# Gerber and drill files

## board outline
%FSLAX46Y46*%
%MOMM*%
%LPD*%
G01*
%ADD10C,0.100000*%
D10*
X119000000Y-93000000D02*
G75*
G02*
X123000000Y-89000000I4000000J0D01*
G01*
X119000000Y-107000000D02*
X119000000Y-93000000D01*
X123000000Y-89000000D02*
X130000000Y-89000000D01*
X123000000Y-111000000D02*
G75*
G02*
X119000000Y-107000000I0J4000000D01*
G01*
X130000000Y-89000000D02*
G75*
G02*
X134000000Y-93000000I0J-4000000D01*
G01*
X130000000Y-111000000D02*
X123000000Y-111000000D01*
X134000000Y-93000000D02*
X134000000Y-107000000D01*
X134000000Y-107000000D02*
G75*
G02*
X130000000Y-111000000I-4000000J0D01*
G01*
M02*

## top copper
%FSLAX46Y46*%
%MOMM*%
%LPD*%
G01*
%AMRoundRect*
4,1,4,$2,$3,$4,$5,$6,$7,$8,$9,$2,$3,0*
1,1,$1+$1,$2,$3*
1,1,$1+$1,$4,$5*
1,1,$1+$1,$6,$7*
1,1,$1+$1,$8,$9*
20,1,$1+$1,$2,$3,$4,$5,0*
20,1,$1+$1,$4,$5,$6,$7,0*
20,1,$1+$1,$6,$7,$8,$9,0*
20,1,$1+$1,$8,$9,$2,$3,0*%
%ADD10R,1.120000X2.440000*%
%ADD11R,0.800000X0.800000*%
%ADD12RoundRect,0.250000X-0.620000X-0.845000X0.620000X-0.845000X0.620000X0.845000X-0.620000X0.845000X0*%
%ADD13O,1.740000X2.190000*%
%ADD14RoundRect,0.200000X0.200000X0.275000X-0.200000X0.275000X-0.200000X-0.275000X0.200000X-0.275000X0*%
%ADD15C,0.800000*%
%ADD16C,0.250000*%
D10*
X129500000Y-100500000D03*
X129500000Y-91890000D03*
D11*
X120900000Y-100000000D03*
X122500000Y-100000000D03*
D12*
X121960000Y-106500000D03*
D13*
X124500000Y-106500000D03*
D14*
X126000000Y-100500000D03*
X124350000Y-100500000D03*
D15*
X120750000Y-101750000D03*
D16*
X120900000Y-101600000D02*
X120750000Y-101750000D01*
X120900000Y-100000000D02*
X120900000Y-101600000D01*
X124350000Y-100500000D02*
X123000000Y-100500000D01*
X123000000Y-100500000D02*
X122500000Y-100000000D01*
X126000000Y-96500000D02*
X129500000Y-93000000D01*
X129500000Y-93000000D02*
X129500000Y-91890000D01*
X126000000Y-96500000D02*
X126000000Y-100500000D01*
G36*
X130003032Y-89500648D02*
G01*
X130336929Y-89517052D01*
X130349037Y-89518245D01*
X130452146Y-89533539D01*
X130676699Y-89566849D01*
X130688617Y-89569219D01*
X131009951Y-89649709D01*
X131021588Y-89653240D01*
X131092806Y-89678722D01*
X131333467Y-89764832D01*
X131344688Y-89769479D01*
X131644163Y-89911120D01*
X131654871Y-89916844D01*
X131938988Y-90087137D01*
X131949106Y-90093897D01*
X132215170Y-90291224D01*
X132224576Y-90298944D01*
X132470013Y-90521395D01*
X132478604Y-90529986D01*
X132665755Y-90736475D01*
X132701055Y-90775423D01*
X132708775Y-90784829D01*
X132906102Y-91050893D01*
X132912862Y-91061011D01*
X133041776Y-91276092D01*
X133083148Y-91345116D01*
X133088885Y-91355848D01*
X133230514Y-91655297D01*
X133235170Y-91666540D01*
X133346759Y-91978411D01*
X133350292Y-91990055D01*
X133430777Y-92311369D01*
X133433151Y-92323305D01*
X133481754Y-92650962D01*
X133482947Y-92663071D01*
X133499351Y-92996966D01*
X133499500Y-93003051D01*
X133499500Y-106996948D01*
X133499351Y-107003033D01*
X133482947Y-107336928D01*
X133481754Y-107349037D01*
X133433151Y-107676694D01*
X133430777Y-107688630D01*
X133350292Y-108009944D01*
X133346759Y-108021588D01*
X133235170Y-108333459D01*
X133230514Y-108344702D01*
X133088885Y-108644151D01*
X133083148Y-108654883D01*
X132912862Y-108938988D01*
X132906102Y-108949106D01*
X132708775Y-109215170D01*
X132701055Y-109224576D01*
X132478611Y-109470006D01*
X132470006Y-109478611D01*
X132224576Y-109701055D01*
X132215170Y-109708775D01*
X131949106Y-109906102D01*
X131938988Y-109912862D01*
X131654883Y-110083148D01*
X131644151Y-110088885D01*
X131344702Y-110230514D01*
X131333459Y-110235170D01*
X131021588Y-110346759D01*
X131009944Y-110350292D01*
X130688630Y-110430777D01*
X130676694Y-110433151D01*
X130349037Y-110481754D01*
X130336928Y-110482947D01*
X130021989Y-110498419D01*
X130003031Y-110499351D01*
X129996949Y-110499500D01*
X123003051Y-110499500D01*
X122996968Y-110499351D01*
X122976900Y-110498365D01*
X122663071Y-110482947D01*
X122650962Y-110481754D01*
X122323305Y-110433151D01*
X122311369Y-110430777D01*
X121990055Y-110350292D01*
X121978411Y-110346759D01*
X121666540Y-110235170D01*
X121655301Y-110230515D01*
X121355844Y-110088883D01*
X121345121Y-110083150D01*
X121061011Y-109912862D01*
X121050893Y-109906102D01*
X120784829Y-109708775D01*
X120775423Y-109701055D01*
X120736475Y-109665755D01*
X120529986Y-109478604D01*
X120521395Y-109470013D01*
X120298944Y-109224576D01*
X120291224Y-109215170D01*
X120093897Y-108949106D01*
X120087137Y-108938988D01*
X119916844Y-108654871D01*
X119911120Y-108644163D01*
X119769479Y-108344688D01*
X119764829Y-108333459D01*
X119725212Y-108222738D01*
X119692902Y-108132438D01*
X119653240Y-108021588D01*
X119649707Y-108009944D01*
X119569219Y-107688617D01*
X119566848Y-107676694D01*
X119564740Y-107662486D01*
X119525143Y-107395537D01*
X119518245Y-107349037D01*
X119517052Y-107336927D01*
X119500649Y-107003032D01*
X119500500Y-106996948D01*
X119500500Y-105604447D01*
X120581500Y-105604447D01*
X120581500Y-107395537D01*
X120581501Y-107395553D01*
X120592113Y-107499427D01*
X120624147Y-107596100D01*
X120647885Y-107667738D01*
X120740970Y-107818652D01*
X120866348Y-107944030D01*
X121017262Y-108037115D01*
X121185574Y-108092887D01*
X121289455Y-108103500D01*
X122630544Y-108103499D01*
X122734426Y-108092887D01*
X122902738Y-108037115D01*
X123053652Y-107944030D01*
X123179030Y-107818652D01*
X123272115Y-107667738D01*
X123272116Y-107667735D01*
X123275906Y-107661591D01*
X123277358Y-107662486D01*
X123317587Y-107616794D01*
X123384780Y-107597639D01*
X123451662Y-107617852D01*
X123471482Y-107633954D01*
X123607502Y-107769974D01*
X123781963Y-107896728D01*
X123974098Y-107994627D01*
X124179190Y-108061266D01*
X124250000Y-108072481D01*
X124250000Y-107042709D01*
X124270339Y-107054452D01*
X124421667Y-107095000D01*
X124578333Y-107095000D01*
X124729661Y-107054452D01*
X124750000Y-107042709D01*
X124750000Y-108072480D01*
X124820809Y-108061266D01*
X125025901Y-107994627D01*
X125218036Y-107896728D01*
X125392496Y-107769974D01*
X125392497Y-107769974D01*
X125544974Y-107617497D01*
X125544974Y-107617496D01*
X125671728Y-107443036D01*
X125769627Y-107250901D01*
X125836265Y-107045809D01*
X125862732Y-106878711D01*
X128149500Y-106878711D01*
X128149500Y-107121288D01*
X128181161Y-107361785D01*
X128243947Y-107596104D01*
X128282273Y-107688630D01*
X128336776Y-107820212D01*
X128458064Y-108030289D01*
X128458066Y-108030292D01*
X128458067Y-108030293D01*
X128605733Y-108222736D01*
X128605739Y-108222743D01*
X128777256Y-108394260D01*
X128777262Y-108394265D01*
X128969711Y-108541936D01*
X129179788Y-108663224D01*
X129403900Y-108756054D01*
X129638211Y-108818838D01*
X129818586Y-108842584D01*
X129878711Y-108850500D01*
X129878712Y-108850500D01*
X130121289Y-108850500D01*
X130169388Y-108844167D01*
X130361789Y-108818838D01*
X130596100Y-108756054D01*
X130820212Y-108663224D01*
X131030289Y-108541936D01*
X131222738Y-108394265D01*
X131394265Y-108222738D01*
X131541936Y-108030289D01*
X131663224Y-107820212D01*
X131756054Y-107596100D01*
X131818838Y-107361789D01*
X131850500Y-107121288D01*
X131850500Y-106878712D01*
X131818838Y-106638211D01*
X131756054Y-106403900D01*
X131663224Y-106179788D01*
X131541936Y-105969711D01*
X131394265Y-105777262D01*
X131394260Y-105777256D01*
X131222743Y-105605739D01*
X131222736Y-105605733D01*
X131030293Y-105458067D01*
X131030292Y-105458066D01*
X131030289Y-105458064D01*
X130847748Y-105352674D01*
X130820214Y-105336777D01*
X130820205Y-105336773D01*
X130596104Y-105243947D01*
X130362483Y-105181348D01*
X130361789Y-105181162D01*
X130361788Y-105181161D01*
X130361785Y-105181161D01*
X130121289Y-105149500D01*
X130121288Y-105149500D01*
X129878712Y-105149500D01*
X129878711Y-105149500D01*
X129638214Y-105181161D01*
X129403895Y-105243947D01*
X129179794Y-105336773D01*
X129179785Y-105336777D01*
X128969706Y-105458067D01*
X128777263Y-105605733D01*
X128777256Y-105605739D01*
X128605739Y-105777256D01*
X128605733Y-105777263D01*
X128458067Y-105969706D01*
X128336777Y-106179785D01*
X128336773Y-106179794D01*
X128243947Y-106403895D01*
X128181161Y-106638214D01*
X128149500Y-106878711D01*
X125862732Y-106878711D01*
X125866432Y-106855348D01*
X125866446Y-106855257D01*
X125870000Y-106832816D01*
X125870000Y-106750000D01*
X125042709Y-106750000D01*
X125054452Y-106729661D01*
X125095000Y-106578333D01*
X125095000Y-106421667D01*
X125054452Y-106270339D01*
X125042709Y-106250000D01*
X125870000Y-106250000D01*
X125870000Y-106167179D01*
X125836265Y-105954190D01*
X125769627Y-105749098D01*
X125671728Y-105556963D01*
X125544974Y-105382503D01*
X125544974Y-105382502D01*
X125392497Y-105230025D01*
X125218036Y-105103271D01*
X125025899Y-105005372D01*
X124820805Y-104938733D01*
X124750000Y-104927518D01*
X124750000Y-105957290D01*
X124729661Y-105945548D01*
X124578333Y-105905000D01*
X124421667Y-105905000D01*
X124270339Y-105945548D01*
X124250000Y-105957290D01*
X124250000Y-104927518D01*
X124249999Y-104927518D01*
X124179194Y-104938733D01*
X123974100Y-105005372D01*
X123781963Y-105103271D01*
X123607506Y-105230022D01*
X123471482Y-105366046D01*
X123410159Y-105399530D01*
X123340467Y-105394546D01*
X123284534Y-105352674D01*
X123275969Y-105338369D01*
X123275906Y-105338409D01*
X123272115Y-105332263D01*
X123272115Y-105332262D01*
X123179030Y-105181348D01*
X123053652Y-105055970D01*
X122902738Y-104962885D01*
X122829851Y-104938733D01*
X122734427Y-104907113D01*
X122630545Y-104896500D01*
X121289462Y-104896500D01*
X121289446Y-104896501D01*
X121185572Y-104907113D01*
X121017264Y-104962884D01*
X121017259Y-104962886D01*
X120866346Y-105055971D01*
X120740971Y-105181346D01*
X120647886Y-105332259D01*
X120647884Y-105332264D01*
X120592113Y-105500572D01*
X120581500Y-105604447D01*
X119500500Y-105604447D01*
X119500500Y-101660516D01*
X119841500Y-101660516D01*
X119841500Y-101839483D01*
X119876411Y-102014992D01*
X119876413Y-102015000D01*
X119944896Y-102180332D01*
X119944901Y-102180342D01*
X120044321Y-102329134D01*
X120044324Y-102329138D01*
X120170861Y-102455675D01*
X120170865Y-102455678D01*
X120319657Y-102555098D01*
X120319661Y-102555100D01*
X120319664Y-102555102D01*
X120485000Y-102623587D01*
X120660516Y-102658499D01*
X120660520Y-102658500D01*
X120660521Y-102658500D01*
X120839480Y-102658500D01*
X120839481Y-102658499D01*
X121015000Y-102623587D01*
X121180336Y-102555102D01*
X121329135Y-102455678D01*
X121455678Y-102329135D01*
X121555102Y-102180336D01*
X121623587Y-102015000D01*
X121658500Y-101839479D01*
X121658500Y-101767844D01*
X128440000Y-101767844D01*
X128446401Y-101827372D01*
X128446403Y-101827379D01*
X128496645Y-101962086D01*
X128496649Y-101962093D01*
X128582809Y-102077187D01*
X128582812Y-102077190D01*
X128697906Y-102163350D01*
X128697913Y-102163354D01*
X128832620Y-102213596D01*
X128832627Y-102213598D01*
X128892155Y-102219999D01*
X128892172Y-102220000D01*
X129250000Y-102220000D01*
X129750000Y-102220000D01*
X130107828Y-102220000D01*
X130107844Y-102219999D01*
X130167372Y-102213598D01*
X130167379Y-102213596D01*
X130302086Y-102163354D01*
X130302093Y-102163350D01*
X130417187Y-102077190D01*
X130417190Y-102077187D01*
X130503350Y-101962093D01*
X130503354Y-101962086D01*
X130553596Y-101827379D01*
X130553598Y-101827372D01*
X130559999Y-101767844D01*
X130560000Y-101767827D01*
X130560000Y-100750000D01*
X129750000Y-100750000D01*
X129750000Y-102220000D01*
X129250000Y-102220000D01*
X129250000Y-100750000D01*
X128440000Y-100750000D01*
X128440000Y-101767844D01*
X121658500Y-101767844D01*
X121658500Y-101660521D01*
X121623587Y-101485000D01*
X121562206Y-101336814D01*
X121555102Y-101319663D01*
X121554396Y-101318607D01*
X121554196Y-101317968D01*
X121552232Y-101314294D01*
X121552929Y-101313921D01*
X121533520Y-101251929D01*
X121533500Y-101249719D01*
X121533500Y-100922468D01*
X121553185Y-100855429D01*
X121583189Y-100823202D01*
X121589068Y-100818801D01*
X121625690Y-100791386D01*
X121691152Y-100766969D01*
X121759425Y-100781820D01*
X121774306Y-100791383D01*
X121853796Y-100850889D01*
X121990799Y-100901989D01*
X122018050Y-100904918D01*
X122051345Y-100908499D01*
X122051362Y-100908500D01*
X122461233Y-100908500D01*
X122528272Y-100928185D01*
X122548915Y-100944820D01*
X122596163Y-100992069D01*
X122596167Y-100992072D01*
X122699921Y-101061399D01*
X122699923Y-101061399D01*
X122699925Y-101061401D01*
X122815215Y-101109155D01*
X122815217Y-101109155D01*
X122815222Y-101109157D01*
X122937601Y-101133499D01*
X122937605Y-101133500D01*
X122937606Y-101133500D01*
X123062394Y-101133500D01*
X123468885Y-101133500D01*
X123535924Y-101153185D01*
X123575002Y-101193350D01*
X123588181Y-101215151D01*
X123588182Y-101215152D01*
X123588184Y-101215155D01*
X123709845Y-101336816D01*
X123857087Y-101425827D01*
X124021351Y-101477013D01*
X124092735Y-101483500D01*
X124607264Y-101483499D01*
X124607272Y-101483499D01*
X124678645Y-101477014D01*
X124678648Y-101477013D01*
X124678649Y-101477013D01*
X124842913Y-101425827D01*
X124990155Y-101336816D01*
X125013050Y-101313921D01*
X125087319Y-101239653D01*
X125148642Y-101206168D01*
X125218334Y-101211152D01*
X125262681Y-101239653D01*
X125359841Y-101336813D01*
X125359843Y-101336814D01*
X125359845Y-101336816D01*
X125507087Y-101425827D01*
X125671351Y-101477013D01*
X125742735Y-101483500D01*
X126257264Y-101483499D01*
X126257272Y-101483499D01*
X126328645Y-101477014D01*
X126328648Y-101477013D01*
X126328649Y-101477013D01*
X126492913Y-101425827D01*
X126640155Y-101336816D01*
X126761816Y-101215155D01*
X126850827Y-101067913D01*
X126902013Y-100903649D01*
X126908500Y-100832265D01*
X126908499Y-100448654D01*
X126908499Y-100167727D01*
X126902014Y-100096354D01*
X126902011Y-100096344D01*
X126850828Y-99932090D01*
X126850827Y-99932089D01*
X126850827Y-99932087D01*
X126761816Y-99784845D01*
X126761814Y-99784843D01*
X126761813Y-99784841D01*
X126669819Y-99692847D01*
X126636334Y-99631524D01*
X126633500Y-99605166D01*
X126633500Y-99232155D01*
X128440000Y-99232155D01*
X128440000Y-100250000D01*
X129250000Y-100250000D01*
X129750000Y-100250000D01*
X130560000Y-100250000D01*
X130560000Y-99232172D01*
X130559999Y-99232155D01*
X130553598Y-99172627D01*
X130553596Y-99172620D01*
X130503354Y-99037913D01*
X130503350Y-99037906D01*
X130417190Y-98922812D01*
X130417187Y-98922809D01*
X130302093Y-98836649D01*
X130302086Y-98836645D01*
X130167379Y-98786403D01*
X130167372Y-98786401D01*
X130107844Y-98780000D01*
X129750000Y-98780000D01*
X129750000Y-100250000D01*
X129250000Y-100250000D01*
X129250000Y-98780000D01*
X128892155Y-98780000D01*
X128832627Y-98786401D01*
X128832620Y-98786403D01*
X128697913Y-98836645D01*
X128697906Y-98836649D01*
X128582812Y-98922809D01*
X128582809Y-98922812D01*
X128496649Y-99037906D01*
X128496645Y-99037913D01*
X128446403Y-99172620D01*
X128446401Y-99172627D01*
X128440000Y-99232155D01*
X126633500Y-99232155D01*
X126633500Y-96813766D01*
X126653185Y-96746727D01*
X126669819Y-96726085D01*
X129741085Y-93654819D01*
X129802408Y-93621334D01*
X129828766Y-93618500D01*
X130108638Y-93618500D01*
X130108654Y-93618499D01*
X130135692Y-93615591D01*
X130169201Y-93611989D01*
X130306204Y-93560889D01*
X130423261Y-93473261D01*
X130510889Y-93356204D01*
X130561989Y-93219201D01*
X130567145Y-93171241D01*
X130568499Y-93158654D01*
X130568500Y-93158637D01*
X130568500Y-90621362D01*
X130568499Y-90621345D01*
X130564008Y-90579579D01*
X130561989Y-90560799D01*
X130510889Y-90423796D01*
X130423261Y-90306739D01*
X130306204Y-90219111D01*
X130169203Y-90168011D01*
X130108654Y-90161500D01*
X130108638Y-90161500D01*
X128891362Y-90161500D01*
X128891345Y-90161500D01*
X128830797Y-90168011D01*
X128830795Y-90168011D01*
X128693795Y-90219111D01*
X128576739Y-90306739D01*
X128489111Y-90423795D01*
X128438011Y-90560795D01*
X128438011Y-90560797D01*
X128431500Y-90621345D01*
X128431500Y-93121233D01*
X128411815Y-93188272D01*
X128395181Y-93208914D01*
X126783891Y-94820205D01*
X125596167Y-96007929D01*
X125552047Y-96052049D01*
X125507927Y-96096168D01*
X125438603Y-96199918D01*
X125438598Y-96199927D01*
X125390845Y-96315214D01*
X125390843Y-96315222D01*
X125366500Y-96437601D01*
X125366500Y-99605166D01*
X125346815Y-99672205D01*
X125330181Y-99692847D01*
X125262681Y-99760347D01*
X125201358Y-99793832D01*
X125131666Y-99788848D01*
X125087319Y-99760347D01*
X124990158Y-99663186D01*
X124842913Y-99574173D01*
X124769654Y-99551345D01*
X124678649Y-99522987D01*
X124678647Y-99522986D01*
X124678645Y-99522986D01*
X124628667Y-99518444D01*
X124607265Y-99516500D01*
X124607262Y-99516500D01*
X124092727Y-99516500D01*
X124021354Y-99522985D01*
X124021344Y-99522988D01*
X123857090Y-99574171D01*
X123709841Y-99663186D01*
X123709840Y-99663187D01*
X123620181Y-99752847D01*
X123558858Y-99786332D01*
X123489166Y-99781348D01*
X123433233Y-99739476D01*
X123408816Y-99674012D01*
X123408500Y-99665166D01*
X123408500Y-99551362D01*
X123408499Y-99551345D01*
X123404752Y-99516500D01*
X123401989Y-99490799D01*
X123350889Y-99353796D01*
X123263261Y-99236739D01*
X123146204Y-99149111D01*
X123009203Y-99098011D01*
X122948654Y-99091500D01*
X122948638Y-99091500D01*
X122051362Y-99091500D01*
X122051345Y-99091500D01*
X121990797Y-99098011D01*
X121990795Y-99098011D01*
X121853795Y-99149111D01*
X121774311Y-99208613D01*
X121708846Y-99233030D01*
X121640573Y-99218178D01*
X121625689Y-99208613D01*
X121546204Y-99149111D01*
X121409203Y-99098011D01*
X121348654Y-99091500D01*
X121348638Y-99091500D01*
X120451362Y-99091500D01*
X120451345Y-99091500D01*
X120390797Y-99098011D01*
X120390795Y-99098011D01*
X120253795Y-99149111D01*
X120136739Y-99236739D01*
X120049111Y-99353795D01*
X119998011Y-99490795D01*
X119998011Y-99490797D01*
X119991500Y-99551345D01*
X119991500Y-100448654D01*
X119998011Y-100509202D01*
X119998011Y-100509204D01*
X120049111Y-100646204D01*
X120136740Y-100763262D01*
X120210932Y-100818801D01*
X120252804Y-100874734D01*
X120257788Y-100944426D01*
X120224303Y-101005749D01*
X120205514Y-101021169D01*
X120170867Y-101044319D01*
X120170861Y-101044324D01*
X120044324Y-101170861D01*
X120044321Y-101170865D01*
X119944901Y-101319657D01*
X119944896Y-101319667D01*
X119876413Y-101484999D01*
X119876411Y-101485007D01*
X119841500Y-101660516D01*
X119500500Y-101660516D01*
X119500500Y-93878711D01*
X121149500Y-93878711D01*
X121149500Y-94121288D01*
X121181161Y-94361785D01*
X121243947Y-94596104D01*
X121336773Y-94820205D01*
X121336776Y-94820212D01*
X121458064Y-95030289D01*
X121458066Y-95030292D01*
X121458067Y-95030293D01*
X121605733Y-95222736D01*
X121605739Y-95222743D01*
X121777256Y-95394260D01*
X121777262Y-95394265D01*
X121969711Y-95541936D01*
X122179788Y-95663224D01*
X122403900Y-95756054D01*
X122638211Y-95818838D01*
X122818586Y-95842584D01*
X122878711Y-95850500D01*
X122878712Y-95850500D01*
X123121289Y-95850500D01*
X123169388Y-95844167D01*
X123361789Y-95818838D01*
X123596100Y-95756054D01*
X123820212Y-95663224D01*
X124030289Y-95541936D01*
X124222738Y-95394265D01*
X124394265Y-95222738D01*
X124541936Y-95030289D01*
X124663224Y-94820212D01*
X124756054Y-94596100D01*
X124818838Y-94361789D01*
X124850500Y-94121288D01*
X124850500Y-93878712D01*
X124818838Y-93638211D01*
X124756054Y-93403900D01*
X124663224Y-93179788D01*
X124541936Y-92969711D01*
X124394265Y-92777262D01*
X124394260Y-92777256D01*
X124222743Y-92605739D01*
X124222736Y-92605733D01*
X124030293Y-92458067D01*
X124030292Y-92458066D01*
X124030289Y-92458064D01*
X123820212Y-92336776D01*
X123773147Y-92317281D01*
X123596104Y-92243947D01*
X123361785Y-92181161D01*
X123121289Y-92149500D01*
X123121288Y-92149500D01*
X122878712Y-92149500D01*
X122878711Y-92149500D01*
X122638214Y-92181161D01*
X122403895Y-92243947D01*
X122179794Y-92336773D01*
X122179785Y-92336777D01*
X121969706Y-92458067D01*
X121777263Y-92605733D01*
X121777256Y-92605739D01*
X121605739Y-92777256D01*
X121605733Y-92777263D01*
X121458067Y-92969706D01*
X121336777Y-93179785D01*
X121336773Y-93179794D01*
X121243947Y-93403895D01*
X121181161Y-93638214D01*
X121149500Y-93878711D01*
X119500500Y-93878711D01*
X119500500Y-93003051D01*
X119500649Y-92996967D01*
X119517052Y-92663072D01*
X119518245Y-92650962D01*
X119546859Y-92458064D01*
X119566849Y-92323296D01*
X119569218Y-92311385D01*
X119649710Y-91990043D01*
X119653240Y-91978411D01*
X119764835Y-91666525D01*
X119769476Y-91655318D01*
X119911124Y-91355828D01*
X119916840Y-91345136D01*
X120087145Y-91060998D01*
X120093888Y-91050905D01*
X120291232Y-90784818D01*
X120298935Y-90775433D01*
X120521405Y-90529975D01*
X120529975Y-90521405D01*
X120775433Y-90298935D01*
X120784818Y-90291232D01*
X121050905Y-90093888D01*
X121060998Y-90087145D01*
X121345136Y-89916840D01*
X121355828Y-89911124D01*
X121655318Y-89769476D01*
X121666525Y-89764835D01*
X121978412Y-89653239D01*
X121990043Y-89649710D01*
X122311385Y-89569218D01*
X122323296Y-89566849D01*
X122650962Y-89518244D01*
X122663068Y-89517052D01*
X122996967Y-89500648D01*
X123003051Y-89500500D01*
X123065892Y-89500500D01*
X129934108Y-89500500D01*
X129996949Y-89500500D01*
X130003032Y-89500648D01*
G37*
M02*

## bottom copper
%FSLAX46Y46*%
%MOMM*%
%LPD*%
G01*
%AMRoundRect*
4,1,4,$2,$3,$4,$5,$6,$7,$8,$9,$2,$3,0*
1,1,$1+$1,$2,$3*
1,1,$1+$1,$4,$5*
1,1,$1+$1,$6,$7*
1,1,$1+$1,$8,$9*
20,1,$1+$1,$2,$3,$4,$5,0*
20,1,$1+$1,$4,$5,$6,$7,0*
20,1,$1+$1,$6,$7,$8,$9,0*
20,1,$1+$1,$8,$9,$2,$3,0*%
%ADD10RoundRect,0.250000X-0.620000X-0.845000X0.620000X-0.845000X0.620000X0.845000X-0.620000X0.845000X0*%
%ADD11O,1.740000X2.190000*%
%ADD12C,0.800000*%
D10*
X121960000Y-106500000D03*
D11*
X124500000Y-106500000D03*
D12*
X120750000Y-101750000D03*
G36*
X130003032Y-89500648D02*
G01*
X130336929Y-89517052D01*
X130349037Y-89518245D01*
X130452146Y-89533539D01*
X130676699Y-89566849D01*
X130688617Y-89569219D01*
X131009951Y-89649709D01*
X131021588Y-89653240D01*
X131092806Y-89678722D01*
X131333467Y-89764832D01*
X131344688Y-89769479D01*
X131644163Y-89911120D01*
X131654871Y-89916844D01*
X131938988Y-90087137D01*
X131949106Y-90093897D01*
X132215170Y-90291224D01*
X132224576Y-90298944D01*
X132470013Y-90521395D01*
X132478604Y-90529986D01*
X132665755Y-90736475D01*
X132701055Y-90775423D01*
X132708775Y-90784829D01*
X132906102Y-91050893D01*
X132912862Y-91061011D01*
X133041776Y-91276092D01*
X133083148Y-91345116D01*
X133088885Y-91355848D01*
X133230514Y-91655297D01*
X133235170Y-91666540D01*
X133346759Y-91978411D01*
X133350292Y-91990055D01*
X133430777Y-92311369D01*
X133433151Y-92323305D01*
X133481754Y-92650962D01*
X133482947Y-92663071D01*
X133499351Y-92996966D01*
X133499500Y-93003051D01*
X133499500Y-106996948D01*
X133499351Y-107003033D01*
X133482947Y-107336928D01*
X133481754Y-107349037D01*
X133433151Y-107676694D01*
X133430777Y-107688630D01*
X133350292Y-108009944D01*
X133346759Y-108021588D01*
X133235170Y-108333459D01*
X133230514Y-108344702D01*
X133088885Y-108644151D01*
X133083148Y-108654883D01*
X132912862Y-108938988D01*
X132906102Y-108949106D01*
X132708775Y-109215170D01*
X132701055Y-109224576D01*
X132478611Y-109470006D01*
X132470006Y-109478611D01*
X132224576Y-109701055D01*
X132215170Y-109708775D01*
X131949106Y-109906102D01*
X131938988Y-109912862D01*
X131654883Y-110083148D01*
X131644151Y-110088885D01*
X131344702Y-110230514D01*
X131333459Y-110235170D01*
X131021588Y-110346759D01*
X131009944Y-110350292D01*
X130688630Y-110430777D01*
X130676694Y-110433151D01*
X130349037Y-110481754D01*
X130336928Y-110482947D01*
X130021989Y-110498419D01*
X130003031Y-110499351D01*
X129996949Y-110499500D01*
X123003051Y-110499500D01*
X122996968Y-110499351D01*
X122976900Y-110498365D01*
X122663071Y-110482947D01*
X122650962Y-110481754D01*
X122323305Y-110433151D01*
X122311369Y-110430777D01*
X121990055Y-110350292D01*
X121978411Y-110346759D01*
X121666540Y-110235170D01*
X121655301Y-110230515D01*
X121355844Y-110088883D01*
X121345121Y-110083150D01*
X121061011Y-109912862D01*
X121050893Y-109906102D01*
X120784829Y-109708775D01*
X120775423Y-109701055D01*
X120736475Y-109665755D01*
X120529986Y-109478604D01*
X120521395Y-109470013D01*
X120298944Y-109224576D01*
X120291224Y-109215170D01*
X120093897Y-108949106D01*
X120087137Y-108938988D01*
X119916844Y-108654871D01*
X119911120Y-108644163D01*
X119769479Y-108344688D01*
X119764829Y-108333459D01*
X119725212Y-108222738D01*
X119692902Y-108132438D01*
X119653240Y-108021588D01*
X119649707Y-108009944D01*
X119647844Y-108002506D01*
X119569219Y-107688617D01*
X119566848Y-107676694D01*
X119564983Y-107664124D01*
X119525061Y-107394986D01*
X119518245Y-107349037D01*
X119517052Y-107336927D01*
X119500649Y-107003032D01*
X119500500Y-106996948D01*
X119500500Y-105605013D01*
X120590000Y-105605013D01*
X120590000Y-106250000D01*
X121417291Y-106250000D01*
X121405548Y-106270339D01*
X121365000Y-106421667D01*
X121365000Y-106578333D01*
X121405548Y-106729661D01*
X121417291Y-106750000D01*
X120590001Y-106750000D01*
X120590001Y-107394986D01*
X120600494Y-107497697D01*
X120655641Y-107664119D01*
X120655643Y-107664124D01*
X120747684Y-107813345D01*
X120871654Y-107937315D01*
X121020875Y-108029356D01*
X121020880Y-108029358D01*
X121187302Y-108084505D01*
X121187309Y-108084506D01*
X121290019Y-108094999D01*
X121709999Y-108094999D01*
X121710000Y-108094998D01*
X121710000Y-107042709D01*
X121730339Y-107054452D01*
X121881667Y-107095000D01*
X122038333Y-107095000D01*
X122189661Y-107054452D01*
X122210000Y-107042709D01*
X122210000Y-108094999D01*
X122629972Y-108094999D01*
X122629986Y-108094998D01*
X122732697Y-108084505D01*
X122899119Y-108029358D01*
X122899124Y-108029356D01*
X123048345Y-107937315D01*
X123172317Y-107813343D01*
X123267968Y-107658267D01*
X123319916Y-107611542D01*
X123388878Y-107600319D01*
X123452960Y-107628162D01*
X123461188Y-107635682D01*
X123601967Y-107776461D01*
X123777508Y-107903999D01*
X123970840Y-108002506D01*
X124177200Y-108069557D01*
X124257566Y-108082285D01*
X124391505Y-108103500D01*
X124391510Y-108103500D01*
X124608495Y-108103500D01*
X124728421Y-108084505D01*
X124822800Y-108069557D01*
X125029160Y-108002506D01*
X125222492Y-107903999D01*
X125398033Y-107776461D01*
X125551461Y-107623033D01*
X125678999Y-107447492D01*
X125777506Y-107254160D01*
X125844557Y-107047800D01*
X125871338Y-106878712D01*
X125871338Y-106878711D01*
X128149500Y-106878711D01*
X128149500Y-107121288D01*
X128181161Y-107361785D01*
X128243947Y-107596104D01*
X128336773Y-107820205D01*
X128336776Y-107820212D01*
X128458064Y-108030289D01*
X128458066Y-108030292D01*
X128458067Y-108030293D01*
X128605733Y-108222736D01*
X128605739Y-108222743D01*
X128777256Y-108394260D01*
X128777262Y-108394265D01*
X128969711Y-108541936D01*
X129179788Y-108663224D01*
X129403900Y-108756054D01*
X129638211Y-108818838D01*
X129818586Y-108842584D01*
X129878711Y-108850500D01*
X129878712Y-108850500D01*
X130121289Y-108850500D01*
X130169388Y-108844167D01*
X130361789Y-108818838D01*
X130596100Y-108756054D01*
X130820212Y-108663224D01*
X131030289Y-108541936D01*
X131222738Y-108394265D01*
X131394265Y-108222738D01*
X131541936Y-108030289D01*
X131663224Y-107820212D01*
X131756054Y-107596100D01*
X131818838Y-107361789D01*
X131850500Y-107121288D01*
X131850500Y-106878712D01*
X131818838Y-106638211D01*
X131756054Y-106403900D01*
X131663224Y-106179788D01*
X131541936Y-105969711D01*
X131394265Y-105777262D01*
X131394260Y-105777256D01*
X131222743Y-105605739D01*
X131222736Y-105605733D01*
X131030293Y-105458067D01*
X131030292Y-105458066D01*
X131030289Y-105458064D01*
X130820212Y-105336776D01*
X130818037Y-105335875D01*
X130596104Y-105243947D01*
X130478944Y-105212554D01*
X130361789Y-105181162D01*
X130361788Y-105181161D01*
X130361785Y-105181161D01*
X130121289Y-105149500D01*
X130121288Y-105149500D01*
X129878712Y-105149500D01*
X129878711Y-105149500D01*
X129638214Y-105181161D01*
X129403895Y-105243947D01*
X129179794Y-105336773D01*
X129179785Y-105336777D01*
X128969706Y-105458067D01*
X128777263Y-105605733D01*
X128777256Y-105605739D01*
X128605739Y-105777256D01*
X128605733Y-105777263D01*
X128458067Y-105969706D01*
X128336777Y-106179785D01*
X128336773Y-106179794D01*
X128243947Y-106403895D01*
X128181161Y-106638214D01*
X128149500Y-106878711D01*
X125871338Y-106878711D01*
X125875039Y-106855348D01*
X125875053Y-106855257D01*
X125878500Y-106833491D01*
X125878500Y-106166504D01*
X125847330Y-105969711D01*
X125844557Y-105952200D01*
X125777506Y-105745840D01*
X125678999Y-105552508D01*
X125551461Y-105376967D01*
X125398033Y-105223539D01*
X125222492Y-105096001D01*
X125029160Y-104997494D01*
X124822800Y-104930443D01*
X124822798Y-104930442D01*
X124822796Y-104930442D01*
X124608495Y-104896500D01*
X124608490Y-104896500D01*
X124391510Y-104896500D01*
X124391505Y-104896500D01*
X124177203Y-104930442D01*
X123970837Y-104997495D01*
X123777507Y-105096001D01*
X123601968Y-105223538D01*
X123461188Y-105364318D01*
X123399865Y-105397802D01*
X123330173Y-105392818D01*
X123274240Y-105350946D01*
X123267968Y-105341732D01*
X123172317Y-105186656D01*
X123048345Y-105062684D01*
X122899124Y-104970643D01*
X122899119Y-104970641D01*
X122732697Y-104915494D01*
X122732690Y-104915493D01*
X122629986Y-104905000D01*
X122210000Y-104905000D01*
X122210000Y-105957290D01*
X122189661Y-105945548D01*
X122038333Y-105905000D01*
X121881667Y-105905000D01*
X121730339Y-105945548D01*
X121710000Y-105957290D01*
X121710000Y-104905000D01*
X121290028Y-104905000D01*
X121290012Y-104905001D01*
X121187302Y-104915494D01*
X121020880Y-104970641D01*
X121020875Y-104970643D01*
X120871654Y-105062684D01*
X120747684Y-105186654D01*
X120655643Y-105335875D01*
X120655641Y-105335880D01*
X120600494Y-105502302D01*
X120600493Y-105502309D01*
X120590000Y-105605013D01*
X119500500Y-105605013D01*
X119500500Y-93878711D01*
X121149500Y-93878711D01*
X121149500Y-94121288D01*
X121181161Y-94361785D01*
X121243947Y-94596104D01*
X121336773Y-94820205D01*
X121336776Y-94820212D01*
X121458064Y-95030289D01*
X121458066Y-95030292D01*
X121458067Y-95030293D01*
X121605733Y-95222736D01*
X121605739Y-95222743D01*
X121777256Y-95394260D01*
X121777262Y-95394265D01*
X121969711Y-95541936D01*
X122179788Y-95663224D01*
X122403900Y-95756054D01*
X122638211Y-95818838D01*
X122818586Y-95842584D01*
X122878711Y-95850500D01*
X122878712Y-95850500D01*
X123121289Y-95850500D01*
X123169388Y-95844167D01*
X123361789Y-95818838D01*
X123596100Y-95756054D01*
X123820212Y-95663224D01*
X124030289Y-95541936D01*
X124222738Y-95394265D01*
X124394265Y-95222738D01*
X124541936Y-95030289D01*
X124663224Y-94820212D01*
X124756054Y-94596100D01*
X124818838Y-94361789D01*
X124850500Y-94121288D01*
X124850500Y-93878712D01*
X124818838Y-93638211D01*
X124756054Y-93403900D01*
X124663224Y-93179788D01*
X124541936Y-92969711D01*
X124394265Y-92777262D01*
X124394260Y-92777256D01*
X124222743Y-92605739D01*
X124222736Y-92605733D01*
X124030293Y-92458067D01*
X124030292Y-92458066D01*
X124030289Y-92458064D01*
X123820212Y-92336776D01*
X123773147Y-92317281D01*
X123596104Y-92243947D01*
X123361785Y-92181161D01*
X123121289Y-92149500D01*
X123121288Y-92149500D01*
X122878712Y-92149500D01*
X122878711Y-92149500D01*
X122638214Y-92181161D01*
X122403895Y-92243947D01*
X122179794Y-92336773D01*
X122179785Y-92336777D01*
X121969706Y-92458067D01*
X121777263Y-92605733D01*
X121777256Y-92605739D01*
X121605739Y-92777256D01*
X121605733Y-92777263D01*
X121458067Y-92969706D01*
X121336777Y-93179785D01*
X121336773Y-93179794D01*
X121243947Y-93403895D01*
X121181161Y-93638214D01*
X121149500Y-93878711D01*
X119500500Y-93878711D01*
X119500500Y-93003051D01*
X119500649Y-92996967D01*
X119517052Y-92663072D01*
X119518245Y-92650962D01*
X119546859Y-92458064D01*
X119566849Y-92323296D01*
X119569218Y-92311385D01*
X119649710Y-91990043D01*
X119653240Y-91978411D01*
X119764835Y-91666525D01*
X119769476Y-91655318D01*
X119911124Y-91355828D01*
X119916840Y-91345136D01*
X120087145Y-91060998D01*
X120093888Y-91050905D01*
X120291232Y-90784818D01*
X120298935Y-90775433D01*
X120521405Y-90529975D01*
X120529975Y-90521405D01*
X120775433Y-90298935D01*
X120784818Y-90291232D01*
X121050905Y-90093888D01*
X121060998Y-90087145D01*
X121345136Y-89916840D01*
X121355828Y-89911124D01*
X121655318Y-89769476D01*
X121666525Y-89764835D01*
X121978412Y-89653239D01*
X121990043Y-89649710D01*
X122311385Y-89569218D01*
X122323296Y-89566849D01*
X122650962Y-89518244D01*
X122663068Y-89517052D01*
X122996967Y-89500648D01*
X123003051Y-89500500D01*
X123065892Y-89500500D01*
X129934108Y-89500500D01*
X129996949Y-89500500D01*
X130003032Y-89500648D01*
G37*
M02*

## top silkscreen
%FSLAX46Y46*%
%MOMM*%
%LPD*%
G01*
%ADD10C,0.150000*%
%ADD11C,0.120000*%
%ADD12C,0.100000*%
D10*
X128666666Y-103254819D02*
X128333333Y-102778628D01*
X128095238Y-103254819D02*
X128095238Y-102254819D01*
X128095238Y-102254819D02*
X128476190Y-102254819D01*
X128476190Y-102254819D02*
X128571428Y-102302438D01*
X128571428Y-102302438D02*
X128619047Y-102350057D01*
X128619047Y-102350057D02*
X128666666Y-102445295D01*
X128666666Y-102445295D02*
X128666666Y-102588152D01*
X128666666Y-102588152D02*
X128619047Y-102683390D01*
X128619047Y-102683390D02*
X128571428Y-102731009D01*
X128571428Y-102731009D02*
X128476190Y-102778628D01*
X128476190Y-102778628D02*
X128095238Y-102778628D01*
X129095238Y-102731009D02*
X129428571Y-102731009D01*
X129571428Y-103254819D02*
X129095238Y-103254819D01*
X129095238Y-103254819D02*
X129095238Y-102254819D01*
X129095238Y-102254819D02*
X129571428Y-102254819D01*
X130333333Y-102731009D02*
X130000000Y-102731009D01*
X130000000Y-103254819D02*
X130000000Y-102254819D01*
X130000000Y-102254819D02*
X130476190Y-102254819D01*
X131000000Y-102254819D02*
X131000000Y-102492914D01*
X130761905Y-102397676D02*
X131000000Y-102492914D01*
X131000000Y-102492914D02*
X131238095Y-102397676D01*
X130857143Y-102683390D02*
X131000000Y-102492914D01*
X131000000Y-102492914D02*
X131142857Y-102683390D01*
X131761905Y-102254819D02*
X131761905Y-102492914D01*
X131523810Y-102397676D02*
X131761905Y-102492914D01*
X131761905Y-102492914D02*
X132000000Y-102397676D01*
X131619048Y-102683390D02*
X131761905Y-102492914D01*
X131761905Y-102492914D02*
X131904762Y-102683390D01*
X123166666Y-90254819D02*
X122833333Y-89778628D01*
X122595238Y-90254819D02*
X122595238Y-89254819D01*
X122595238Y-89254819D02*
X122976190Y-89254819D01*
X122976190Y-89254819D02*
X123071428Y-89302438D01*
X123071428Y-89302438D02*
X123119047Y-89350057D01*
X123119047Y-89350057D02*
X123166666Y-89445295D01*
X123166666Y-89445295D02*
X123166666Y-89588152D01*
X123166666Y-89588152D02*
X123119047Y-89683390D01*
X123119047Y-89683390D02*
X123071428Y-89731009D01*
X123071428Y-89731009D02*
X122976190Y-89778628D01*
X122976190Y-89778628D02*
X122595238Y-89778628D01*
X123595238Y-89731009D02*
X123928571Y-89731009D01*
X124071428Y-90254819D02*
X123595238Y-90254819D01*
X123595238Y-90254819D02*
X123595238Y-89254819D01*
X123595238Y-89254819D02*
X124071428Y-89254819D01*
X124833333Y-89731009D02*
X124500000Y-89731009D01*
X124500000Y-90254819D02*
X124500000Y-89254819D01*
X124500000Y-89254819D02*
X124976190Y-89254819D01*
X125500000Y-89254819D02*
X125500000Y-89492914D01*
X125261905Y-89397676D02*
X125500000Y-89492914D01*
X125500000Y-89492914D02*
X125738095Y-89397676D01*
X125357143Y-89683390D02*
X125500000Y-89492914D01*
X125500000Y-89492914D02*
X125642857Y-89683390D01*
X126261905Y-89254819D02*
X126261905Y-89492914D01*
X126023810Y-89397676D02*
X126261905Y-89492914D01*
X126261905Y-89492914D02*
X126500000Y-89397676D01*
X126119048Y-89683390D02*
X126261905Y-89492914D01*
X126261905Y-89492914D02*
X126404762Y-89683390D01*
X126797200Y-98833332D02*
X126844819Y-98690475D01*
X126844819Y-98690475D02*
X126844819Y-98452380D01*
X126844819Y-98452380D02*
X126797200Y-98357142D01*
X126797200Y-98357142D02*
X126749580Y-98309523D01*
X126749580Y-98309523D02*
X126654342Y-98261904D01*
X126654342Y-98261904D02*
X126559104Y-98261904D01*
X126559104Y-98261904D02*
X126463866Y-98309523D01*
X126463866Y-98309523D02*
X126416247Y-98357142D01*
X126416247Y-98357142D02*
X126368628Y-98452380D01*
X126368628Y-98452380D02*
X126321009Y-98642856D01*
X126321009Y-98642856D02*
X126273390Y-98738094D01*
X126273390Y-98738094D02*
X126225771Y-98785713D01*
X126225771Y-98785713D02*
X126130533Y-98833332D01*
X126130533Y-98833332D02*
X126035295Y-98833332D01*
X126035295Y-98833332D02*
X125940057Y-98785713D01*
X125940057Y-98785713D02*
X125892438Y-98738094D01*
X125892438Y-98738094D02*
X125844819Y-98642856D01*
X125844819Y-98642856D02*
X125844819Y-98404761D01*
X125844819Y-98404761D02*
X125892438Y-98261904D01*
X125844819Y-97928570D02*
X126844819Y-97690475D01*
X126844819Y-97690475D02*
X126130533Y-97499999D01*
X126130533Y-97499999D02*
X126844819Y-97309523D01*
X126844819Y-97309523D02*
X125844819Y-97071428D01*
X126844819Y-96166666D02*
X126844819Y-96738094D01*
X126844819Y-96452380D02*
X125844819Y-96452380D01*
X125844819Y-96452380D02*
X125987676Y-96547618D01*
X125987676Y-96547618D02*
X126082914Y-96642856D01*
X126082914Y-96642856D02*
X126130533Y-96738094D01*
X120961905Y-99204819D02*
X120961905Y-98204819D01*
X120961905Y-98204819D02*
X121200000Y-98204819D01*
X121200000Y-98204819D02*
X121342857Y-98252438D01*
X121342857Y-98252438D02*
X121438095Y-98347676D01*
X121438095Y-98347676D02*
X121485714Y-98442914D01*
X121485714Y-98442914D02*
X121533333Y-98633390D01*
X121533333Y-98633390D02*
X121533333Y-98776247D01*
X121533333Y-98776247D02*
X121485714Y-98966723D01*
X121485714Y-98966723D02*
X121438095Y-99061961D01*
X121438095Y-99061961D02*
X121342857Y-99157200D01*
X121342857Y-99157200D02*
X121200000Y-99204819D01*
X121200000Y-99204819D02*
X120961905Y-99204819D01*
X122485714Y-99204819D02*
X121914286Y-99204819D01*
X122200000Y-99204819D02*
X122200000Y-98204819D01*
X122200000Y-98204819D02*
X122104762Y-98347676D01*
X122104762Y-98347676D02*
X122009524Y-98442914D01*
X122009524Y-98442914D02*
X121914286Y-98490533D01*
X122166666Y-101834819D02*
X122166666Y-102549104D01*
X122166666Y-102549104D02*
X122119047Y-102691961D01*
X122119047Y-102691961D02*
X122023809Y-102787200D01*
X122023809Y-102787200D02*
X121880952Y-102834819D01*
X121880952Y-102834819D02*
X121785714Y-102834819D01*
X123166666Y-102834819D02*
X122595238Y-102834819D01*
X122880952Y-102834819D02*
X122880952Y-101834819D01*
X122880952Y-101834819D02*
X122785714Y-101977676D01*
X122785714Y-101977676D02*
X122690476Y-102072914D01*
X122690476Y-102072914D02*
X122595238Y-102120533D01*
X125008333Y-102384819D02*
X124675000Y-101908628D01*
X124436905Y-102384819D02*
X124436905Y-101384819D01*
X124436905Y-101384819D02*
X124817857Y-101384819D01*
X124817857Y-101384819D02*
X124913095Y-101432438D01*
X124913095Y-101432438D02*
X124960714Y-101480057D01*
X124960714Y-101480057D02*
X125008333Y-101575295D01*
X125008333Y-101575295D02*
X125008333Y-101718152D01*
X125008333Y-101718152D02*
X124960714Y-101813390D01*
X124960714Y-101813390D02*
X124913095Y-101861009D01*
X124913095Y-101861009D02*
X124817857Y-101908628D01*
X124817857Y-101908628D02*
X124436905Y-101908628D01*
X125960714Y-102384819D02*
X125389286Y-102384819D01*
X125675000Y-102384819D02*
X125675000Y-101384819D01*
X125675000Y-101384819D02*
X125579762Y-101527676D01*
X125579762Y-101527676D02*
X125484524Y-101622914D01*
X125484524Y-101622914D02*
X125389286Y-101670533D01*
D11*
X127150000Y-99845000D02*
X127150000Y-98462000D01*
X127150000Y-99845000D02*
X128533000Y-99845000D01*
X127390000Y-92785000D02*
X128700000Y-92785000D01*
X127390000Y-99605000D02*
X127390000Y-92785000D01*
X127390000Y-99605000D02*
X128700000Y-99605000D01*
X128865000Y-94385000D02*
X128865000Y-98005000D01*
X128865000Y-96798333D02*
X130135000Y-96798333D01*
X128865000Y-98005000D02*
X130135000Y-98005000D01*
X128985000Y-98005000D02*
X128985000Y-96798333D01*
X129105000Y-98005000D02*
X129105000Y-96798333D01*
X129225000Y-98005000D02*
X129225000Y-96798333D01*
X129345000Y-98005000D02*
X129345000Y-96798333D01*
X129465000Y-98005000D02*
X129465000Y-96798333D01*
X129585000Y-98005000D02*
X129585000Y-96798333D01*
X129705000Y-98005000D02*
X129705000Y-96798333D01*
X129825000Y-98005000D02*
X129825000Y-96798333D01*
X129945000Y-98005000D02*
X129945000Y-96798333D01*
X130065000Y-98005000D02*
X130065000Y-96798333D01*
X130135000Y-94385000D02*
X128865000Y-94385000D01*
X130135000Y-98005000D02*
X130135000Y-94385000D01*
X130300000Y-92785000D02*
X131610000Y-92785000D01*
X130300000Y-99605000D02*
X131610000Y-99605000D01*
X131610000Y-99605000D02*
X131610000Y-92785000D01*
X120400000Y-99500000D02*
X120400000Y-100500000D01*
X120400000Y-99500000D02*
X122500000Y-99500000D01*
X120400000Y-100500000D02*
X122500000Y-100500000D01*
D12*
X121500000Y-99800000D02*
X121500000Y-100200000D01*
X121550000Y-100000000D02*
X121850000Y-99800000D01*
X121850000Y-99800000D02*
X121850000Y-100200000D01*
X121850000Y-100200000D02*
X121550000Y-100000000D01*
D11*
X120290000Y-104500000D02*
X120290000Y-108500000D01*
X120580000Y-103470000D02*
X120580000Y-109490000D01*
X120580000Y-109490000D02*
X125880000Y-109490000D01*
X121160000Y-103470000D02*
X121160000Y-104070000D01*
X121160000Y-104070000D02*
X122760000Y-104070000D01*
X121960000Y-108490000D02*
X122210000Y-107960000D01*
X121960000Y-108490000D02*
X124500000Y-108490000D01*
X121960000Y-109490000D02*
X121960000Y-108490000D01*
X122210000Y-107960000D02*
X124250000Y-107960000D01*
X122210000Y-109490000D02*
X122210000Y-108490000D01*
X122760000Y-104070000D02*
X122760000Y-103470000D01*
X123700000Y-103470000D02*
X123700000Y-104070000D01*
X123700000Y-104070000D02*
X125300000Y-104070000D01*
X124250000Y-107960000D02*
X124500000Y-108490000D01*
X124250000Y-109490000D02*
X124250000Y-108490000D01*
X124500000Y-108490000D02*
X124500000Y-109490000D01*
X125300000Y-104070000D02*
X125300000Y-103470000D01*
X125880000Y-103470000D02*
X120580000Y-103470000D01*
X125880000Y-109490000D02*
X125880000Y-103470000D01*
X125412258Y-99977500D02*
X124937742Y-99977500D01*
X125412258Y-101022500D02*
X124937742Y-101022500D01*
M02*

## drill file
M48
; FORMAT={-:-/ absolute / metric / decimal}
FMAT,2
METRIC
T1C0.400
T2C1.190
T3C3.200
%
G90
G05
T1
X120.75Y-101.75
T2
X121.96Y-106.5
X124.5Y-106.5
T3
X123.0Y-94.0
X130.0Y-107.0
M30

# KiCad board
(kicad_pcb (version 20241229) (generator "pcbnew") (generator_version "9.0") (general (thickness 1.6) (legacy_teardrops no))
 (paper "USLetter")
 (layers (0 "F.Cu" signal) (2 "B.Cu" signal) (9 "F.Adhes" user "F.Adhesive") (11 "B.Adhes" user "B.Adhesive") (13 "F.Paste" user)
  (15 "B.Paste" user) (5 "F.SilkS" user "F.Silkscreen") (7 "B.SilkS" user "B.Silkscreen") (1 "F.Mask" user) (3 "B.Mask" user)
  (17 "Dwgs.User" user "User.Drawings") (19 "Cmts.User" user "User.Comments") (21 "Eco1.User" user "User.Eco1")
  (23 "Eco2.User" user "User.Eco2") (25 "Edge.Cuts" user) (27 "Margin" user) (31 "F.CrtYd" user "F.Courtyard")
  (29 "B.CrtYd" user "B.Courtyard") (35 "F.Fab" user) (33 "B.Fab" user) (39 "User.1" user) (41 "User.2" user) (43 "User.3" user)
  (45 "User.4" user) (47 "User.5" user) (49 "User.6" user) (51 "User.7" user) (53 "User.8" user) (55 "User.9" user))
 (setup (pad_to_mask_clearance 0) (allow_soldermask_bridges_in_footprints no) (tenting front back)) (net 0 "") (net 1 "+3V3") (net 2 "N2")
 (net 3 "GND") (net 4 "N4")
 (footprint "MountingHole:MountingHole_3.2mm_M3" (layer "F.Cu") (at 130 107)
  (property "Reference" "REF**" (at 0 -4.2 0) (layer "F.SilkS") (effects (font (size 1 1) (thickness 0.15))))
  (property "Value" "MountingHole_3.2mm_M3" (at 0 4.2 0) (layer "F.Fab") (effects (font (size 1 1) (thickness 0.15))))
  (pad "" np_thru_hole circle (at 0 0) (size 3.2 3.2) (drill 3.2) (layers "*.Cu" "*.Mask")))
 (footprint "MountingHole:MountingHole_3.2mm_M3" (layer "F.Cu") (at 123 94)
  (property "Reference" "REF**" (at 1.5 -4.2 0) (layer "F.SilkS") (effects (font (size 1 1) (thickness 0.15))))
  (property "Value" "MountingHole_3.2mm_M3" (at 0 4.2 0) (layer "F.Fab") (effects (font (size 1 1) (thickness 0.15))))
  (pad "" np_thru_hole circle (at 0 0) (size 3.2 3.2) (drill 3.2) (layers "*.Cu" "*.Mask")))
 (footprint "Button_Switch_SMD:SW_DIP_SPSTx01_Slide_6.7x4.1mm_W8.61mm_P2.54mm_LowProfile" (layer "F.Cu") (at 129.5 96.195 90)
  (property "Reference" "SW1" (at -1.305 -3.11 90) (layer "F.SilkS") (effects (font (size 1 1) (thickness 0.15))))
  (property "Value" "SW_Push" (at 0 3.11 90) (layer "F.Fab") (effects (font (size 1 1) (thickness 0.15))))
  (fp_line (start -3.65 -2.35) (end -2.267 -2.35) (stroke (width 0.12) (type solid)) (layer "F.SilkS"))
  (fp_line (start -3.65 -2.35) (end -3.65 -0.967) (stroke (width 0.12) (type solid)) (layer "F.SilkS"))
  (fp_line (start 3.41 -2.11) (end 3.41 -0.8) (stroke (width 0.12) (type solid)) (layer "F.SilkS"))
  (fp_line (start -3.41 -2.11) (end 3.41 -2.11) (stroke (width 0.12) (type solid)) (layer "F.SilkS"))
  (fp_line (start -3.41 -2.11) (end -3.41 -0.8) (stroke (width 0.12) (type solid)) (layer "F.SilkS"))
  (fp_line (start 1.81 -0.635) (end -1.81 -0.635) (stroke (width 0.12) (type solid)) (layer "F.SilkS"))
  (fp_line (start -0.603333 -0.635) (end -0.603333 0.635) (stroke (width 0.12) (type solid)) (layer "F.SilkS"))
  (fp_line (start -1.81 -0.635) (end -1.81 0.635) (stroke (width 0.12) (type solid)) (layer "F.SilkS"))
  (fp_line (start -1.81 -0.515) (end -0.603333 -0.515) (stroke (width 0.12) (type solid)) (layer "F.SilkS"))
  (fp_line (start -1.81 -0.395) (end -0.603333 -0.395) (stroke (width 0.12) (type solid)) (layer "F.SilkS"))
  (fp_line (start -1.81 -0.275) (end -0.603333 -0.275) (stroke (width 0.12) (type solid)) (layer "F.SilkS"))
  (fp_line (start -1.81 -0.155) (end -0.603333 -0.155) (stroke (width 0.12) (type solid)) (layer "F.SilkS"))
  (fp_line (start -1.81 -0.035) (end -0.603333 -0.035) (stroke (width 0.12) (type solid)) (layer "F.SilkS"))
  (fp_line (start -1.81 0.085) (end -0.603333 0.085) (stroke (width 0.12) (type solid)) (layer "F.SilkS"))
  (fp_line (start -1.81 0.205) (end -0.603333 0.205) (stroke (width 0.12) (type solid)) (layer "F.SilkS"))
  (fp_line (start -1.81 0.325) (end -0.603333 0.325) (stroke (width 0.12) (type solid)) (layer "F.SilkS"))
  (fp_line (start -1.81 0.445) (end -0.603333 0.445) (stroke (width 0.12) (type solid)) (layer "F.SilkS"))
  (fp_line (start -1.81 0.565) (end -0.603333 0.565) (stroke (width 0.12) (type solid)) (layer "F.SilkS"))
  (fp_line (start 1.81 0.635) (end 1.81 -0.635) (stroke (width 0.12) (type solid)) (layer "F.SilkS"))
  (fp_line (start -1.81 0.635) (end 1.81 0.635) (stroke (width 0.12) (type solid)) (layer "F.SilkS"))
  (fp_line (start 3.41 0.8) (end 3.41 2.11) (stroke (width 0.12) (type solid)) (layer "F.SilkS"))
  (fp_line (start -3.41 0.8) (end -3.41 2.11) (stroke (width 0.12) (type solid)) (layer "F.SilkS"))
  (fp_line (start -3.41 2.11) (end 3.41 2.11) (stroke (width 0.12) (type solid)) (layer "F.SilkS"))
  (pad "1" smd rect (at -4.305 0 90) (size 2.44 1.12) (layers "F.Cu" "F.Mask" "F.Paste") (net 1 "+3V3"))
  (pad "2" smd rect (at 4.305 0 90) (size 2.44 1.12) (layers "F.Cu" "F.Mask" "F.Paste") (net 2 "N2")))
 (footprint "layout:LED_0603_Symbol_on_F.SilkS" (layer "F.Cu") (at 121.7 100)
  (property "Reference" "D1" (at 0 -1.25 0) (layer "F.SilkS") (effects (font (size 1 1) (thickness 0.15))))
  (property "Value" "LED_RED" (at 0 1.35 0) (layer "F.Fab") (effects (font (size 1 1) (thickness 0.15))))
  (fp_line (start -1.3 -0.5) (end -1.3 0.5) (stroke (width 0.12) (type solid)) (layer "F.SilkS"))
  (fp_line (start -1.3 -0.5) (end 0.8 -0.5) (stroke (width 0.12) (type solid)) (layer "F.SilkS"))
  (fp_line (start -1.3 0.5) (end 0.8 0.5) (stroke (width 0.12) (type solid)) (layer "F.SilkS"))
  (fp_line (start -0.2 -0.2) (end -0.2 0.2) (stroke (width 0.1) (type solid)) (layer "F.SilkS"))
  (fp_line (start -0.15 0) (end 0.15 -0.2) (stroke (width 0.1) (type solid)) (layer "F.SilkS"))
  (fp_line (start 0.15 -0.2) (end 0.15 0.2) (stroke (width 0.1) (type solid)) (layer "F.SilkS"))
  (fp_line (start 0.15 0.2) (end -0.15 0) (stroke (width 0.1) (type solid)) (layer "F.SilkS"))
  (pad "1" smd rect (at -0.8 0 180) (size 0.8 0.8) (layers "F.Cu" "F.Mask" "F.Paste") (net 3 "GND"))
  (pad "2" smd rect (at 0.8 0 180) (size 0.8 0.8) (layers "F.Cu" "F.Mask" "F.Paste") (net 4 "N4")))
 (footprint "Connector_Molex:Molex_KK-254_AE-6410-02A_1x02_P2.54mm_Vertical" (layer "F.Cu") (at 121.96 106.5)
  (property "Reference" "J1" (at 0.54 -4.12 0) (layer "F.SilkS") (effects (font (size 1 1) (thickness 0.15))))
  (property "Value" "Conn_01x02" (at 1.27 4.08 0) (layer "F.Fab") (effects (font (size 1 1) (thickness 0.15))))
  (fp_line (start -1.67 -2) (end -1.67 2) (stroke (width 0.12) (type solid)) (layer "F.SilkS"))
  (fp_line (start -1.38 -3.03) (end -1.38 2.99) (stroke (width 0.12) (type solid)) (layer "F.SilkS"))
  (fp_line (start -1.38 2.99) (end 3.92 2.99) (stroke (width 0.12) (type solid)) (layer "F.SilkS"))
  (fp_line (start -0.8 -3.03) (end -0.8 -2.43) (stroke (width 0.12) (type solid)) (layer "F.SilkS"))
  (fp_line (start -0.8 -2.43) (end 0.8 -2.43) (stroke (width 0.12) (type solid)) (layer "F.SilkS"))
  (fp_line (start 0 1.99) (end 0.25 1.46) (stroke (width 0.12) (type solid)) (layer "F.SilkS"))
  (fp_line (start 0 1.99) (end 2.54 1.99) (stroke (width 0.12) (type solid)) (layer "F.SilkS"))
  (fp_line (start 0 2.99) (end 0 1.99) (stroke (width 0.12) (type solid)) (layer "F.SilkS"))
  (fp_line (start 0.25 1.46) (end 2.29 1.46) (stroke (width 0.12) (type solid)) (layer "F.SilkS"))
  (fp_line (start 0.25 2.99) (end 0.25 1.99) (stroke (width 0.12) (type solid)) (layer "F.SilkS"))
  (fp_line (start 0.8 -2.43) (end 0.8 -3.03) (stroke (width 0.12) (type solid)) (layer "F.SilkS"))
  (fp_line (start 1.74 -3.03) (end 1.74 -2.43) (stroke (width 0.12) (type solid)) (layer "F.SilkS"))
  (fp_line (start 1.74 -2.43) (end 3.34 -2.43) (stroke (width 0.12) (type solid)) (layer "F.SilkS"))
  (fp_line (start 2.29 1.46) (end 2.54 1.99) (stroke (width 0.12) (type solid)) (layer "F.SilkS"))
  (fp_line (start 2.29 2.99) (end 2.29 1.99) (stroke (width 0.12) (type solid)) (layer "F.SilkS"))
  (fp_line (start 2.54 1.99) (end 2.54 2.99) (stroke (width 0.12) (type solid)) (layer "F.SilkS"))
  (fp_line (start 3.34 -2.43) (end 3.34 -3.03) (stroke (width 0.12) (type solid)) (layer "F.SilkS"))
  (fp_line (start 3.92 -3.03) (end -1.38 -3.03) (stroke (width 0.12) (type solid)) (layer "F.SilkS"))
  (fp_line (start 3.92 2.99) (end 3.92 -3.03) (stroke (width 0.12) (type solid)) (layer "F.SilkS"))
  (pad "1" thru_hole roundrect (at 0 0) (size 1.74 2.19) (drill 1.19) (layers "*.Cu" "*.Mask") (remove_unused_layers no)
   (roundrect_rratio 0.143678) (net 3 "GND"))
  (pad "2" thru_hole oval (at 2.54 0) (size 1.74 2.19) (drill 1.19) (layers "*.Cu" "*.Mask") (remove_unused_layers no) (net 1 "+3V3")))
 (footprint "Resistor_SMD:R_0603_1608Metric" (layer "F.Cu") (at 125.175 100.5 180)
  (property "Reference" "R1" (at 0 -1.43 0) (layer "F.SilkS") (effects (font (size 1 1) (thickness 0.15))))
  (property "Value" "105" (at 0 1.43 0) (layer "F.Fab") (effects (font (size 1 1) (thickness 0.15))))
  (fp_line (start -0.237258 0.5225) (end 0.237258 0.5225) (stroke (width 0.12) (type solid)) (layer "F.SilkS"))
  (fp_line (start -0.237258 -0.5225) (end 0.237258 -0.5225) (stroke (width 0.12) (type solid)) (layer "F.SilkS"))
  (pad "1" smd roundrect (at -0.825 0 180) (size 0.8 0.95) (layers "F.Cu" "F.Mask" "F.Paste") (roundrect_rratio 0.25) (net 2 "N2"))
  (pad "2" smd roundrect (at 0.825 0 180) (size 0.8 0.95) (layers "F.Cu" "F.Mask" "F.Paste") (roundrect_rratio 0.25) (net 4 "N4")))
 (gr_arc (start 119 93) (mid 120.171573 90.171573) (end 123 89) (stroke (width 0.1) (type default)) (layer "Edge.Cuts"))
 (gr_line (start 119 107) (end 119 93) (stroke (width 0.1) (type default)) (layer "Edge.Cuts"))
 (gr_line (start 123 89) (end 130 89) (stroke (width 0.1) (type default)) (layer "Edge.Cuts"))
 (gr_arc (start 123 111) (mid 120.171573 109.828427) (end 119 107) (stroke (width 0.1) (type default)) (layer "Edge.Cuts"))
 (gr_arc (start 130 89) (mid 132.828427 90.171573) (end 134 93) (stroke (width 0.1) (type default)) (layer "Edge.Cuts"))
 (gr_line (start 130 111) (end 123 111) (stroke (width 0.1) (type default)) (layer "Edge.Cuts"))
 (gr_line (start 134 93) (end 134 107) (stroke (width 0.1) (type default)) (layer "Edge.Cuts"))
 (gr_arc (start 134 107) (mid 132.828427 109.828427) (end 130 111) (stroke (width 0.1) (type default)) (layer "Edge.Cuts"))
 (segment (start 120.9 101.6) (end 120.75 101.75) (width 0.25) (layer "F.Cu") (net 3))
 (segment (start 120.9 100) (end 120.9 101.6) (width 0.25) (layer "F.Cu") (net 3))
 (via (at 120.75 101.75) (size 0.8) (drill 0.4) (layers "F.Cu" "B.Cu") (free yes) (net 3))
 (segment (start 124.35 100.5) (end 123 100.5) (width 0.25) (layer "F.Cu") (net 4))
 (segment (start 123 100.5) (end 122.5 100) (width 0.25) (layer "F.Cu") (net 4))
 (segment (start 126 96.5) (end 129.5 93) (width 0.25) (layer "F.Cu") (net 2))
 (segment (start 129.5 93) (end 129.5 91.89) (width 0.25) (layer "F.Cu") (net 2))
 (segment (start 126 96.5) (end 126 100.5) (width 0.25) (layer "F.Cu") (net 2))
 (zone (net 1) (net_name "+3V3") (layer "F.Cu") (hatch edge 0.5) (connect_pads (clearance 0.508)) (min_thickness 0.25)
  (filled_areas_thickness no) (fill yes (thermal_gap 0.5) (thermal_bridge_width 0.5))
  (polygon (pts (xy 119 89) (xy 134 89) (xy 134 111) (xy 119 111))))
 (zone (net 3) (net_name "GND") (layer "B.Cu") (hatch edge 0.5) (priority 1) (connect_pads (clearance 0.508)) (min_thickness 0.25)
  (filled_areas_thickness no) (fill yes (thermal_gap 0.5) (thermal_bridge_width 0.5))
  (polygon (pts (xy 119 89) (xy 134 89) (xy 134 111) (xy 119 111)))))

